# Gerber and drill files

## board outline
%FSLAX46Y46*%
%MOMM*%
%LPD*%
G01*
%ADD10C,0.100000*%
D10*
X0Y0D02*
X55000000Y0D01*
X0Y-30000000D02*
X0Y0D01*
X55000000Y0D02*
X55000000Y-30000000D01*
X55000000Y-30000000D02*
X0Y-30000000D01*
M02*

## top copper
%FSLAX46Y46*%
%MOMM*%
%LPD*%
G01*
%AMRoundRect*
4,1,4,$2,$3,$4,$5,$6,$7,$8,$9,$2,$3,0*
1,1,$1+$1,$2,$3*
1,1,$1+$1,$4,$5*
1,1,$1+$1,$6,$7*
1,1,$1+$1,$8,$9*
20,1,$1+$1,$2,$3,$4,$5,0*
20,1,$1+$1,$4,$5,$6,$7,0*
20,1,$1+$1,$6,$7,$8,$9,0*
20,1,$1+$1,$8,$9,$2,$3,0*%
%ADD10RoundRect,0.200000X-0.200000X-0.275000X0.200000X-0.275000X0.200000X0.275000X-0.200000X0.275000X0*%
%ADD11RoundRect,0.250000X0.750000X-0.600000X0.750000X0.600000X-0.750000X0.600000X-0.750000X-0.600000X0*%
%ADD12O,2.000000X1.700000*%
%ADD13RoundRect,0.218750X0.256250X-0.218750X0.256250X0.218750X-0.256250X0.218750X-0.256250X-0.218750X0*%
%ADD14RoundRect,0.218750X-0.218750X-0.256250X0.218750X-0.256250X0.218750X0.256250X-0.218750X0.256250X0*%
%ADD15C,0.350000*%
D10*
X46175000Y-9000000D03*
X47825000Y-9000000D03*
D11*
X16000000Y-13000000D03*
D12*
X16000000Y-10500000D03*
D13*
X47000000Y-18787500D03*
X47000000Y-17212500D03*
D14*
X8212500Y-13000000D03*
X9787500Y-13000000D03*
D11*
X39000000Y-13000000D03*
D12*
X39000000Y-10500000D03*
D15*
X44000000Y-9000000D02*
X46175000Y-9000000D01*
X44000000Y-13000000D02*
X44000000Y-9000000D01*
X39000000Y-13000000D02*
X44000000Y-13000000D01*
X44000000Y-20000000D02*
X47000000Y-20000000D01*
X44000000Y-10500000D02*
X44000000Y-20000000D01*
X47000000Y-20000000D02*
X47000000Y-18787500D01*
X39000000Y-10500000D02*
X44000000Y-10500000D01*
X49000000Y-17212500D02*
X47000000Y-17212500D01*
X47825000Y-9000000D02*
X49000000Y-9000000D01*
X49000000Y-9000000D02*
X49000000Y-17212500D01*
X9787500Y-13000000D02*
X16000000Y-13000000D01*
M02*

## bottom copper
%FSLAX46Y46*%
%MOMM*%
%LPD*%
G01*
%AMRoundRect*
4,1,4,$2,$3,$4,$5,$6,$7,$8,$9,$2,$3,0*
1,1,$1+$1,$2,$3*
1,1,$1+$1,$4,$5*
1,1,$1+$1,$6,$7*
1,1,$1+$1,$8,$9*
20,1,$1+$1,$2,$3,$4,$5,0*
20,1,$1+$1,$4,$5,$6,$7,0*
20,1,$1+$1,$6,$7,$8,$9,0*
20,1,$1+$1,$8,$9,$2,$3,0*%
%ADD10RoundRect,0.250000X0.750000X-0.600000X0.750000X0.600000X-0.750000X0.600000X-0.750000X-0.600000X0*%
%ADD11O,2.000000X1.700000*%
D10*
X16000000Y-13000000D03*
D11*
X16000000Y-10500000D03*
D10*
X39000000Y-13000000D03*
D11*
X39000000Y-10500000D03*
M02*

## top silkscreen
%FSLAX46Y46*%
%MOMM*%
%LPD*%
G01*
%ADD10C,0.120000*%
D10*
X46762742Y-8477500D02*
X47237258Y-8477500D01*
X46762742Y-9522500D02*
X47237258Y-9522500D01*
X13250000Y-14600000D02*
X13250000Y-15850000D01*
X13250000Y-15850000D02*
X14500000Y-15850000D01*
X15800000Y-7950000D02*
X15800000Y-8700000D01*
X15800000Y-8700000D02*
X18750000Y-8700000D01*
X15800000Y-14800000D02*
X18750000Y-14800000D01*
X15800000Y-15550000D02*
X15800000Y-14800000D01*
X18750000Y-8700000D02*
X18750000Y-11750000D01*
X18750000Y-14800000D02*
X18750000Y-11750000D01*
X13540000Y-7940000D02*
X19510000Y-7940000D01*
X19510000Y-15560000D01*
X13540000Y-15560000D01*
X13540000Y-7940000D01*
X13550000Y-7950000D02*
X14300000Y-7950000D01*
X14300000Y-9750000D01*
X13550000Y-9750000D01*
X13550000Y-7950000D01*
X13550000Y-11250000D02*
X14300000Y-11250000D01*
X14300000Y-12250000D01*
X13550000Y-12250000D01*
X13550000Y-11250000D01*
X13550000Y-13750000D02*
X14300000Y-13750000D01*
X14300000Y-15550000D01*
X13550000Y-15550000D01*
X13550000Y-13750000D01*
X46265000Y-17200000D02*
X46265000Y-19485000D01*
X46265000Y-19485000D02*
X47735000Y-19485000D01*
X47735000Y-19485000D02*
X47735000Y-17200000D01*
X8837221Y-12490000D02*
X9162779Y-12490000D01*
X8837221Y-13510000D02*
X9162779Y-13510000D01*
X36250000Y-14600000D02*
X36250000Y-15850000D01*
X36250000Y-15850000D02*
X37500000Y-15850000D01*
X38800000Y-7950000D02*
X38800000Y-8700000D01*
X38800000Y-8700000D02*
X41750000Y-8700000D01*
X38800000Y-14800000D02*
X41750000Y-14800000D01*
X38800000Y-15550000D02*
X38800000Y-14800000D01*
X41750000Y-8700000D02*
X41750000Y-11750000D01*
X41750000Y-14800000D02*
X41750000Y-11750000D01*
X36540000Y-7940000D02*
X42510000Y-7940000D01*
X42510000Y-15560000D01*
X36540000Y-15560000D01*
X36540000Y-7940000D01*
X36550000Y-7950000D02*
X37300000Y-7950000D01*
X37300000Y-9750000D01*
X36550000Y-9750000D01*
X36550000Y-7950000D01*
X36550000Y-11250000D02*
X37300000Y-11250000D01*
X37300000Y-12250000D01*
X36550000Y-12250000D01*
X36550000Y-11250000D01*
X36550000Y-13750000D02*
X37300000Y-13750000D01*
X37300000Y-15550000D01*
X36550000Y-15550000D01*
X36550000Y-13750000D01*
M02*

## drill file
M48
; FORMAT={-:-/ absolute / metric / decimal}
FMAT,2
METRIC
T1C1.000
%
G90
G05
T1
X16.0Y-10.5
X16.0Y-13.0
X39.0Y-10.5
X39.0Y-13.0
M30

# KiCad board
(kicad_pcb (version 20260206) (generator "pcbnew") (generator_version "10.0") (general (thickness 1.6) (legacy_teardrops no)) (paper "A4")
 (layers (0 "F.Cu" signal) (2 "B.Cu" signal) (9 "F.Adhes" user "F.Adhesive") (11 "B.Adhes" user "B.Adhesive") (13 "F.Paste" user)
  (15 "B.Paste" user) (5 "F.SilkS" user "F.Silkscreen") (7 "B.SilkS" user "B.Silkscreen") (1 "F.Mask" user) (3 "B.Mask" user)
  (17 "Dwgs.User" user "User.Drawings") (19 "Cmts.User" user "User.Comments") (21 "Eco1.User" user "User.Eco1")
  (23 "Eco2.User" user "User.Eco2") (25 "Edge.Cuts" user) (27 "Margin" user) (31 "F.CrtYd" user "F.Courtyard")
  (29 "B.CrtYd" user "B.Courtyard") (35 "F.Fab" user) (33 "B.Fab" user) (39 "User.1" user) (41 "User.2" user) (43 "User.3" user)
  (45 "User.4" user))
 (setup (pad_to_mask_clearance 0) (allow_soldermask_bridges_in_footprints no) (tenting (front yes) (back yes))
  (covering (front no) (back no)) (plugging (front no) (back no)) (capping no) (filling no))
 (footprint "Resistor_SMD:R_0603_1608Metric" (layer "F.Cu") (at 47 9)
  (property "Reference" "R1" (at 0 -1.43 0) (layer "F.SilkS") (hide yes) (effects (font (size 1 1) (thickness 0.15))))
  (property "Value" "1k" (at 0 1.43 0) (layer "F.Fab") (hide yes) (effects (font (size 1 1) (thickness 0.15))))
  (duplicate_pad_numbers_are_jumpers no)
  (fp_line (start -0.237258 -0.5225) (end 0.237258 -0.5225) (stroke (width 0.12) (type solid)) (layer "F.SilkS"))
  (fp_line (start -0.237258 0.5225) (end 0.237258 0.5225) (stroke (width 0.12) (type solid)) (layer "F.SilkS"))
  (pad "1" smd roundrect (at -0.825 0) (size 0.8 0.95) (layers "F.Cu" "F.Mask" "F.Paste") (roundrect_rratio 0.25) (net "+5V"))
  (pad "2" smd roundrect (at 0.825 0) (size 0.8 0.95) (layers "F.Cu" "F.Mask" "F.Paste") (roundrect_rratio 0.25) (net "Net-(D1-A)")))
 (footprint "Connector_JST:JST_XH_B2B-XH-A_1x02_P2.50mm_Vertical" (layer "F.Cu") (at 16 13 90)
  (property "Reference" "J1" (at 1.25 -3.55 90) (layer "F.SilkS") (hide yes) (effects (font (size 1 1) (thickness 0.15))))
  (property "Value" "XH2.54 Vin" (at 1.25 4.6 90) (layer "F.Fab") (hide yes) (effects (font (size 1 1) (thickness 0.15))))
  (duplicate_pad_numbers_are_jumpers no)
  (fp_line (start -1.6 -2.75) (end -2.85 -2.75) (stroke (width 0.12) (type solid)) (layer "F.SilkS"))
  (fp_line (start -2.85 -2.75) (end -2.85 -1.5) (stroke (width 0.12) (type solid)) (layer "F.SilkS"))
  (fp_line (start 5.05 -0.2) (end 4.3 -0.2) (stroke (width 0.12) (type solid)) (layer "F.SilkS"))
  (fp_line (start 4.3 -0.2) (end 4.3 2.75) (stroke (width 0.12) (type solid)) (layer "F.SilkS"))
  (fp_line (start -1.8 -0.2) (end -1.8 2.75) (stroke (width 0.12) (type solid)) (layer "F.SilkS"))
  (fp_line (start -2.55 -0.2) (end -1.8 -0.2) (stroke (width 0.12) (type solid)) (layer "F.SilkS"))
  (fp_line (start 4.3 2.75) (end 1.25 2.75) (stroke (width 0.12) (type solid)) (layer "F.SilkS"))
  (fp_line (start -1.8 2.75) (end 1.25 2.75) (stroke (width 0.12) (type solid)) (layer "F.SilkS"))
  (fp_rect (start -2.56 -2.46) (end 5.06 3.51) (stroke (width 0.12) (type solid)) (fill no) (layer "F.SilkS"))
  (fp_rect (start 3.25 -2.45) (end 5.05 -1.7) (stroke (width 0.12) (type solid)) (fill no) (layer "F.SilkS"))
  (fp_rect (start 0.75 -2.45) (end 1.75 -1.7) (stroke (width 0.12) (type solid)) (fill no) (layer "F.SilkS"))
  (fp_rect (start -2.55 -2.45) (end -0.75 -1.7) (stroke (width 0.12) (type solid)) (fill no) (layer "F.SilkS"))
  (pad "1" thru_hole roundrect (at 0 0 90) (size 1.7 2) (drill 1) (layers "*.Cu" "*.Mask") (remove_unused_layers no)
   (roundrect_rratio 0.147059) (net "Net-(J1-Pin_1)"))
  (pad "2" thru_hole oval (at 2.5 0 90) (size 1.7 2) (drill 1) (layers "*.Cu" "*.Mask") (remove_unused_layers no) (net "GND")))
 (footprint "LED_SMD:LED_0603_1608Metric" (layer "F.Cu") (at 47 18 90)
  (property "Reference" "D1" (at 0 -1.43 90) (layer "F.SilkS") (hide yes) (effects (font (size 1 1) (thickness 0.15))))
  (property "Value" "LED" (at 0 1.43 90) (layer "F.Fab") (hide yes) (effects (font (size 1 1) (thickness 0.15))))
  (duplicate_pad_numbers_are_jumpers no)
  (fp_line (start 0.8 -0.735) (end -1.485 -0.735) (stroke (width 0.12) (type solid)) (layer "F.SilkS"))
  (fp_line (start -1.485 -0.735) (end -1.485 0.735) (stroke (width 0.12) (type solid)) (layer "F.SilkS"))
  (fp_line (start -1.485 0.735) (end 0.8 0.735) (stroke (width 0.12) (type solid)) (layer "F.SilkS"))
  (pad "1" smd roundrect (at -0.7875 0 90) (size 0.875 0.95) (layers "F.Cu" "F.Mask" "F.Paste") (roundrect_rratio 0.25) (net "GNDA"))
  (pad "2" smd roundrect (at 0.7875 0 90) (size 0.875 0.95) (layers "F.Cu" "F.Mask" "F.Paste") (roundrect_rratio 0.25) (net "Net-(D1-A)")))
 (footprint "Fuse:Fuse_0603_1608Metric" (layer "F.Cu") (at 9 13)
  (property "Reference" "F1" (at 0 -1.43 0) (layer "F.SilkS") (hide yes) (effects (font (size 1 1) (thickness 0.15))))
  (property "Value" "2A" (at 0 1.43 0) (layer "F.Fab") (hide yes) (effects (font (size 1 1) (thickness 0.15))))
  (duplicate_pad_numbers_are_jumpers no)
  (fp_line (start -0.162779 -0.51) (end 0.162779 -0.51) (stroke (width 0.12) (type solid)) (layer "F.SilkS"))
  (fp_line (start -0.162779 0.51) (end 0.162779 0.51) (stroke (width 0.12) (type solid)) (layer "F.SilkS"))
  (pad "1" smd roundrect (at -0.7875 0) (size 0.875 0.95) (layers "F.Cu" "F.Mask" "F.Paste") (roundrect_rratio 0.25) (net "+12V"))
  (pad "2" smd roundrect (at 0.7875 0) (size 0.875 0.95) (layers "F.Cu" "F.Mask" "F.Paste") (roundrect_rratio 0.25) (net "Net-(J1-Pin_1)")))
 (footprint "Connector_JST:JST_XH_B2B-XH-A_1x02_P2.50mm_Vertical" (layer "F.Cu") (at 39 13 90)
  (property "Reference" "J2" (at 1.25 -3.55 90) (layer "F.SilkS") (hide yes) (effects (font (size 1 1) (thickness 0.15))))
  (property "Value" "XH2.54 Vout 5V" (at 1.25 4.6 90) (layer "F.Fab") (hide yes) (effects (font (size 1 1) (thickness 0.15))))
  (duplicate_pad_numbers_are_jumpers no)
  (fp_line (start -1.6 -2.75) (end -2.85 -2.75) (stroke (width 0.12) (type solid)) (layer "F.SilkS"))
  (fp_line (start -2.85 -2.75) (end -2.85 -1.5) (stroke (width 0.12) (type solid)) (layer "F.SilkS"))
  (fp_line (start 5.05 -0.2) (end 4.3 -0.2) (stroke (width 0.12) (type solid)) (layer "F.SilkS"))
  (fp_line (start 4.3 -0.2) (end 4.3 2.75) (stroke (width 0.12) (type solid)) (layer "F.SilkS"))
  (fp_line (start -1.8 -0.2) (end -1.8 2.75) (stroke (width 0.12) (type solid)) (layer "F.SilkS"))
  (fp_line (start -2.55 -0.2) (end -1.8 -0.2) (stroke (width 0.12) (type solid)) (layer "F.SilkS"))
  (fp_line (start 4.3 2.75) (end 1.25 2.75) (stroke (width 0.12) (type solid)) (layer "F.SilkS"))
  (fp_line (start -1.8 2.75) (end 1.25 2.75) (stroke (width 0.12) (type solid)) (layer "F.SilkS"))
  (fp_rect (start -2.56 -2.46) (end 5.06 3.51) (stroke (width 0.12) (type solid)) (fill no) (layer "F.SilkS"))
  (fp_rect (start 3.25 -2.45) (end 5.05 -1.7) (stroke (width 0.12) (type solid)) (fill no) (layer "F.SilkS"))
  (fp_rect (start 0.75 -2.45) (end 1.75 -1.7) (stroke (width 0.12) (type solid)) (fill no) (layer "F.SilkS"))
  (fp_rect (start -2.55 -2.45) (end -0.75 -1.7) (stroke (width 0.12) (type solid)) (fill no) (layer "F.SilkS"))
  (pad "1" thru_hole roundrect (at 0 0 90) (size 1.7 2) (drill 1) (layers "*.Cu" "*.Mask") (remove_unused_layers no)
   (roundrect_rratio 0.147059) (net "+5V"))
  (pad "2" thru_hole oval (at 2.5 0 90) (size 1.7 2) (drill 1) (layers "*.Cu" "*.Mask") (remove_unused_layers no) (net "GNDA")))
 (gr_line (start 0 0) (end 55 0) (stroke (width 0.1) (type default)) (layer "Edge.Cuts"))
 (gr_line (start 0 30) (end 0 0) (stroke (width 0.1) (type default)) (layer "Edge.Cuts"))
 (gr_line (start 55 0) (end 55 30) (stroke (width 0.1) (type default)) (layer "Edge.Cuts"))
 (gr_line (start 55 30) (end 0 30) (stroke (width 0.1) (type default)) (layer "Edge.Cuts"))
 (segment (start 44 9) (end 46.175 9) (width 0.35) (layer "F.Cu") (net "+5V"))
 (segment (start 44 13) (end 44 9) (width 0.35) (layer "F.Cu") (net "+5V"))
 (segment (start 39 13) (end 44 13) (width 0.35) (layer "F.Cu") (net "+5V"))
 (segment (start 44 20) (end 47 20) (width 0.35) (layer "F.Cu") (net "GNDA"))
 (segment (start 44 10.5) (end 44 20) (width 0.35) (layer "F.Cu") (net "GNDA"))
 (segment (start 47 20) (end 47 18.7875) (width 0.35) (layer "F.Cu") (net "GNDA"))
 (segment (start 39 10.5) (end 44 10.5) (width 0.35) (layer "F.Cu") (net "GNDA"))
 (segment (start 49 17.2125) (end 47 17.2125) (width 0.35) (layer "F.Cu") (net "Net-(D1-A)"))
 (segment (start 47.825 9) (end 49 9) (width 0.35) (layer "F.Cu") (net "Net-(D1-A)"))
 (segment (start 49 9) (end 49 17.2125) (width 0.35) (layer "F.Cu") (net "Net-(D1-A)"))
 (segment (start 9.7875 13) (end 16 13) (width 0.35) (layer "F.Cu") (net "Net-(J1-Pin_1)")))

